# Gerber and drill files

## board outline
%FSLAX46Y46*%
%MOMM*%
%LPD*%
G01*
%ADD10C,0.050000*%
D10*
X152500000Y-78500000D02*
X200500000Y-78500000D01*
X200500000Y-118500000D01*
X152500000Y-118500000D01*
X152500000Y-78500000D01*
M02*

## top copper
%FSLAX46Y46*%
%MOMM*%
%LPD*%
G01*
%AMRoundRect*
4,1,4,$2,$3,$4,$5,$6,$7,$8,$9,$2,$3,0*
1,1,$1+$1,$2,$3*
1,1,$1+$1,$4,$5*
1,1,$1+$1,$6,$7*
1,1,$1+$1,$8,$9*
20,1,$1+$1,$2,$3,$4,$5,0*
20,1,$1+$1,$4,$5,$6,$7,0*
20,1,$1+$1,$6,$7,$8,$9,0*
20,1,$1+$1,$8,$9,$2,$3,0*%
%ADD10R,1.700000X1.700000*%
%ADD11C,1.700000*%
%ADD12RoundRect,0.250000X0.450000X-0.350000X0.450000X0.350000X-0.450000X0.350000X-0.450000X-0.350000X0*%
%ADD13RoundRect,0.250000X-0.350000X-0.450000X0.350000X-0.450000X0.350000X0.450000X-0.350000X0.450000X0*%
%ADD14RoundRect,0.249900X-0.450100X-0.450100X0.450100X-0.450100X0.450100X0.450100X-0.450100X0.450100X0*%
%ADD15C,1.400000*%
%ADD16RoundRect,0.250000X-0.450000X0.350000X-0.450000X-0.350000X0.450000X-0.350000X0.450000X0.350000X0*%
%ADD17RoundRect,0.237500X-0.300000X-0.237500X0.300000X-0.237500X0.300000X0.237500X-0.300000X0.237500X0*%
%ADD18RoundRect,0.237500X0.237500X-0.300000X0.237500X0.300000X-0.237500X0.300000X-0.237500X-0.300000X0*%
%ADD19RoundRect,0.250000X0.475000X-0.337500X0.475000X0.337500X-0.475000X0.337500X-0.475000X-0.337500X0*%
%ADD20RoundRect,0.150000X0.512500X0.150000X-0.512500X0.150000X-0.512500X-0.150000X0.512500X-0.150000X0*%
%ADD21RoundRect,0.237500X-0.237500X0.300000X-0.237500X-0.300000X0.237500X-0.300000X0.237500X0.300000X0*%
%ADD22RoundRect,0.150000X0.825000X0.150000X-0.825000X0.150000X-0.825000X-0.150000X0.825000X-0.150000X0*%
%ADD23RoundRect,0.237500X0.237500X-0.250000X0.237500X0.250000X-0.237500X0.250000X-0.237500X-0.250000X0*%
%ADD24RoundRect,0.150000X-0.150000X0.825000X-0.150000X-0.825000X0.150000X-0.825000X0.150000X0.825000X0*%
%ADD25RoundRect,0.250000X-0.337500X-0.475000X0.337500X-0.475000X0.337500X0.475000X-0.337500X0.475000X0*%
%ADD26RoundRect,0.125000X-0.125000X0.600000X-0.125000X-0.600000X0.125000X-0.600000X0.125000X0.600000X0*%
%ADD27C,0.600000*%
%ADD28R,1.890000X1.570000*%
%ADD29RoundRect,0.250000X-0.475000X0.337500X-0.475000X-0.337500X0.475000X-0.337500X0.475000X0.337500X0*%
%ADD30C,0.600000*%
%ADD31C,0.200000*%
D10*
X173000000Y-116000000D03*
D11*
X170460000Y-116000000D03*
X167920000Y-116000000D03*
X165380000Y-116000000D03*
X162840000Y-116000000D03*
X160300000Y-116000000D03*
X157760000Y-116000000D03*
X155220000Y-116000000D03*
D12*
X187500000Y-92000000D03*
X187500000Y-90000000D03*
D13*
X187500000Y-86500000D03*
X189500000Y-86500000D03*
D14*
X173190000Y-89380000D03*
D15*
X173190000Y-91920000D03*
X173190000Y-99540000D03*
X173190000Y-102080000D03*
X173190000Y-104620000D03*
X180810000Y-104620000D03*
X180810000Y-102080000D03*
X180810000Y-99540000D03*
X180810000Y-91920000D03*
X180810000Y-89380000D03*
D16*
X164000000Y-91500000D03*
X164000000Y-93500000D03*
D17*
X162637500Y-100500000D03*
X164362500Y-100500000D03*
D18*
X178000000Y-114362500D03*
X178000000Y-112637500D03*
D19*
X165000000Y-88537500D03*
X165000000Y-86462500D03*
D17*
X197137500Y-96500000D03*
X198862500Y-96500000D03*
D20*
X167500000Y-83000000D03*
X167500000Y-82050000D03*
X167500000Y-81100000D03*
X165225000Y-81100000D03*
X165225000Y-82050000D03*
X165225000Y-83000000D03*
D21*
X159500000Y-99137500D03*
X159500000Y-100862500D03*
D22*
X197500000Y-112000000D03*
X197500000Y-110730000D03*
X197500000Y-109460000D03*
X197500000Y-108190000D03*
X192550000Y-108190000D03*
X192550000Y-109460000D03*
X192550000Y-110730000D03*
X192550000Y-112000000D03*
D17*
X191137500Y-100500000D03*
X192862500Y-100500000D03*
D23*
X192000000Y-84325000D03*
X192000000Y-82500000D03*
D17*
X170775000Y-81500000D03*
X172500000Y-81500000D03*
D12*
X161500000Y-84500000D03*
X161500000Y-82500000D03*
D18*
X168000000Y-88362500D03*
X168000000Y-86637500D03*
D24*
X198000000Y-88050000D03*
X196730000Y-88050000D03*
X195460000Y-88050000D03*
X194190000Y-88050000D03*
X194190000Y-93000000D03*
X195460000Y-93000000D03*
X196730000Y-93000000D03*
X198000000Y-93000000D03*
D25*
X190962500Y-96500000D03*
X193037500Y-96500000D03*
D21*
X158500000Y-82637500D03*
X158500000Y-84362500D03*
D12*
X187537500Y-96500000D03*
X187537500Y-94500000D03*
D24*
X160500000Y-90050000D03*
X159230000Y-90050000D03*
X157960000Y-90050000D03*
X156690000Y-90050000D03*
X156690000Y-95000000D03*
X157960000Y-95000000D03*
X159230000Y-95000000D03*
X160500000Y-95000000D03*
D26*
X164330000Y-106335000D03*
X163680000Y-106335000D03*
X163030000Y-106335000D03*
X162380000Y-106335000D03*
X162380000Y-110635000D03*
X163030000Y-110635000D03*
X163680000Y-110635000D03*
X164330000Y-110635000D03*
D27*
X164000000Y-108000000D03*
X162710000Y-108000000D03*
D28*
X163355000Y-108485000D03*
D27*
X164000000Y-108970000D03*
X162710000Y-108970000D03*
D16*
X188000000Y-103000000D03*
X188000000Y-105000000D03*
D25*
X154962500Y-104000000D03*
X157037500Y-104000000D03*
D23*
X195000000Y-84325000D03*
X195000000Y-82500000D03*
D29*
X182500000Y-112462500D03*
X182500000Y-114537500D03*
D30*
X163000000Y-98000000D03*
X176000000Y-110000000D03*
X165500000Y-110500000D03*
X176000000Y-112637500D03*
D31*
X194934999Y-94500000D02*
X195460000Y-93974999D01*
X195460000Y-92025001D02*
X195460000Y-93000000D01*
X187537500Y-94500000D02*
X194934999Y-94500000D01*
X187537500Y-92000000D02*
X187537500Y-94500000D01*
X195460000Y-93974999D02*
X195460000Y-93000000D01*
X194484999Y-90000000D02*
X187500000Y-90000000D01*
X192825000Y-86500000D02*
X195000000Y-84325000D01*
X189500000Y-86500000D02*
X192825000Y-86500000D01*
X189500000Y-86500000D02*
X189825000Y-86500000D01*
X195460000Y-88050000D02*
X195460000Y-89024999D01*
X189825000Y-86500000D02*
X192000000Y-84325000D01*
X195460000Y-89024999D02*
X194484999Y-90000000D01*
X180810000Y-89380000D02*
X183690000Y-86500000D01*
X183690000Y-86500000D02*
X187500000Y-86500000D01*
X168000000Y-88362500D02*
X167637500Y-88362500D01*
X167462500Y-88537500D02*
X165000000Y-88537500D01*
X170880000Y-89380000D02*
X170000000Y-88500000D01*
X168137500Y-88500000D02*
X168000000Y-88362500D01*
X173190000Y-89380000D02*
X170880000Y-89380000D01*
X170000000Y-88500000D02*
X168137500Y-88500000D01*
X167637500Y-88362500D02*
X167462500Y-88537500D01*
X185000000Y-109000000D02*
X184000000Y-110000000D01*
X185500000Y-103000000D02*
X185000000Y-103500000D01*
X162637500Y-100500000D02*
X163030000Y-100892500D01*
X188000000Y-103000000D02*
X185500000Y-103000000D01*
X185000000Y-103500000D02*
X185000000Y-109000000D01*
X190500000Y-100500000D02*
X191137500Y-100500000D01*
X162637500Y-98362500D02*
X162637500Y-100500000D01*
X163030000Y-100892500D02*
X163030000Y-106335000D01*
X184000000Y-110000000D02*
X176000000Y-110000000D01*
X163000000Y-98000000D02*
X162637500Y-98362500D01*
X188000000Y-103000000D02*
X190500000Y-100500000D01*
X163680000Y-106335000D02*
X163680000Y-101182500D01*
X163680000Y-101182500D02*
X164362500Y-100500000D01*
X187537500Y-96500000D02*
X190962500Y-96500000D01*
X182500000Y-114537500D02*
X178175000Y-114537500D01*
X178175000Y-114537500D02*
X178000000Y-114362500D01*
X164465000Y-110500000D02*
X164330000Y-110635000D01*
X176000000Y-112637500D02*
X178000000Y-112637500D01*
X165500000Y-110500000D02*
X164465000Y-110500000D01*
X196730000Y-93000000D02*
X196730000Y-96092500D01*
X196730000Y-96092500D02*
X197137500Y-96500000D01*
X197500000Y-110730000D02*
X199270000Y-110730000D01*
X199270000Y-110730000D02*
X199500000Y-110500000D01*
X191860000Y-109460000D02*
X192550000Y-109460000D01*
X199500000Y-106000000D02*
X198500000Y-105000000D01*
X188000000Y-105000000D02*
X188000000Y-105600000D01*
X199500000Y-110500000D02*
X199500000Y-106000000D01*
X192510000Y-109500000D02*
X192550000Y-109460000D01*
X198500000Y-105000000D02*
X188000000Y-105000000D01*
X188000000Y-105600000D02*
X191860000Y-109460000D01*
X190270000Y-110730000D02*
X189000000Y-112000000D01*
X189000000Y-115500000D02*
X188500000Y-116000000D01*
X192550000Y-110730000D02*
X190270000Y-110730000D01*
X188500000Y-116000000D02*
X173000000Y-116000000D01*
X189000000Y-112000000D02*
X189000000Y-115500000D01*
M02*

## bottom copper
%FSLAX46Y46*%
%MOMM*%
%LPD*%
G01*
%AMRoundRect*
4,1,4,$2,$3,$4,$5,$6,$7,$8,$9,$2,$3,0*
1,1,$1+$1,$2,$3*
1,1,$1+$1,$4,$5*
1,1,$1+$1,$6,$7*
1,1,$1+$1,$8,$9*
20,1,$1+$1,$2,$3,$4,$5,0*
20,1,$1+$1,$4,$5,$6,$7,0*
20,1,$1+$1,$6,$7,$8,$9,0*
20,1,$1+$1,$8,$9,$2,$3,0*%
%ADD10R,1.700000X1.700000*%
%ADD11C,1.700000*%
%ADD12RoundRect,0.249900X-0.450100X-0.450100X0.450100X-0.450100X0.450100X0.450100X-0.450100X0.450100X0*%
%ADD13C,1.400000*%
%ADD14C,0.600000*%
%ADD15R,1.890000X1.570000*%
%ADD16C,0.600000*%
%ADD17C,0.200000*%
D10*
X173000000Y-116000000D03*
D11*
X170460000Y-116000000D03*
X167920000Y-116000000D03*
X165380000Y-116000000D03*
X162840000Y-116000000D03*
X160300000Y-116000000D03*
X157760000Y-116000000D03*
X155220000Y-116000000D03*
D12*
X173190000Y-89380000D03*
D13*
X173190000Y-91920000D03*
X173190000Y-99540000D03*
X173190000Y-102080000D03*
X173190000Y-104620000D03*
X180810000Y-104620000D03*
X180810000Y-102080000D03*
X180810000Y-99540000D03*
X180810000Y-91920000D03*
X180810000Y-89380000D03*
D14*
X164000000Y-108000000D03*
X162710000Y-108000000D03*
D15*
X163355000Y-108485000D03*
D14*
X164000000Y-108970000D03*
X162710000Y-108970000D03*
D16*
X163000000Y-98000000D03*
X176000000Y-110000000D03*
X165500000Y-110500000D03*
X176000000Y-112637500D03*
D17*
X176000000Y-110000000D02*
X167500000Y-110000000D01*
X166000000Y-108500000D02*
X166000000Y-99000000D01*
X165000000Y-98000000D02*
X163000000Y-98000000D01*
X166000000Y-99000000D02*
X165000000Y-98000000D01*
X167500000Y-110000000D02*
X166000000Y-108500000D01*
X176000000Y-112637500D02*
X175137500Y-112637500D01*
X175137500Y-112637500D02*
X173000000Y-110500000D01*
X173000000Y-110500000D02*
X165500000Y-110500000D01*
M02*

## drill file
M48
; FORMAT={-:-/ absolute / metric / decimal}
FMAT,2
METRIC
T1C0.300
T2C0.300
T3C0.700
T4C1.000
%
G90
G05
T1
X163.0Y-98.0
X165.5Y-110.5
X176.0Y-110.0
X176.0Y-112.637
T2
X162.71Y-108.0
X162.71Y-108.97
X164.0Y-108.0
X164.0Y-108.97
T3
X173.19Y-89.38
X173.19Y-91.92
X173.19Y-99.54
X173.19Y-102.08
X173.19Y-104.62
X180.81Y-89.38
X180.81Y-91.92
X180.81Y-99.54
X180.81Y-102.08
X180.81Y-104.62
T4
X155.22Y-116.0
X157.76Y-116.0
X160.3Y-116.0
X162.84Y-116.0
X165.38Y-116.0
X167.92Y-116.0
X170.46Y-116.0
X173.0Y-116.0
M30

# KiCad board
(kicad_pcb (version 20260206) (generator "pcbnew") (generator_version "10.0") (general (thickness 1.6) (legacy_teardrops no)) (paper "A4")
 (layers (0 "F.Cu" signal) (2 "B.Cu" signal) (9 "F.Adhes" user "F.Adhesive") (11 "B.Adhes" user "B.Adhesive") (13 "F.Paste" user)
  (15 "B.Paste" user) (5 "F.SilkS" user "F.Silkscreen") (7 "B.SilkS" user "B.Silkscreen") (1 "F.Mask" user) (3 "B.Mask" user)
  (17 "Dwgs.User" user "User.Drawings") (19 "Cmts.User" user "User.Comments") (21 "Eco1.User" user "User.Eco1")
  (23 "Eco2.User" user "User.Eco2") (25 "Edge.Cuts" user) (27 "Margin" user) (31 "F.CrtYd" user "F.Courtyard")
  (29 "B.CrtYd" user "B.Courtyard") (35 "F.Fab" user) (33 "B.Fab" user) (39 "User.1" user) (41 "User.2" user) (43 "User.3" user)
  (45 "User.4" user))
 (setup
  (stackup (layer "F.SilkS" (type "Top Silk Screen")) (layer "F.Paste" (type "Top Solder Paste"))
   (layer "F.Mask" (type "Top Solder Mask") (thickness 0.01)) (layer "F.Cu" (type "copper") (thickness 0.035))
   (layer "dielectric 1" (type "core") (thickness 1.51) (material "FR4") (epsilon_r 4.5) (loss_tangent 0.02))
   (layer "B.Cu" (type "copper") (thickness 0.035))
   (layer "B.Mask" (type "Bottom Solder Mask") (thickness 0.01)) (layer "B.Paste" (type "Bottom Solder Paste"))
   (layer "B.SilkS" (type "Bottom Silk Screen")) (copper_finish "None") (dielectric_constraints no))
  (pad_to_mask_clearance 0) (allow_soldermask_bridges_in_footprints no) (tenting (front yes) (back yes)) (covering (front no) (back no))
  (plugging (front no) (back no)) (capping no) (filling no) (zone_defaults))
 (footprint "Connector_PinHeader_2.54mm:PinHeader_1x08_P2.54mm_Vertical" (layer "F.Cu") (at 173 116 -90)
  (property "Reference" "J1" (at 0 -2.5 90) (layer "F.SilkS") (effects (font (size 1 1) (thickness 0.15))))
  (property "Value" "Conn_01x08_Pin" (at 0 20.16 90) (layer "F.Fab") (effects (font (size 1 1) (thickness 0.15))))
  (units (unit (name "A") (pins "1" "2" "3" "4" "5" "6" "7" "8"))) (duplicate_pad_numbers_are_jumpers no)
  (pad "1" thru_hole rect (at 0 0 270) (size 1.7 1.7) (drill 1) (layers "*.Cu" "*.Mask") (remove_unused_layers no) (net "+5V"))
  (pad "2" thru_hole circle (at 0 2.54 270) (size 1.7 1.7) (drill 1) (layers "*.Cu" "*.Mask") (remove_unused_layers no) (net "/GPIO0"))
  (pad "3" thru_hole circle (at 0 5.08 270) (size 1.7 1.7) (drill 1) (layers "*.Cu" "*.Mask") (remove_unused_layers no) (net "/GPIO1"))
  (pad "4" thru_hole circle (at 0 7.62 270) (size 1.7 1.7) (drill 1) (layers "*.Cu" "*.Mask") (remove_unused_layers no) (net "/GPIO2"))
  (pad "5" thru_hole circle (at 0 10.16 270) (size 1.7 1.7) (drill 1) (layers "*.Cu" "*.Mask") (remove_unused_layers no) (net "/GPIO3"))
  (pad "6" thru_hole circle (at 0 12.7 270) (size 1.7 1.7) (drill 1) (layers "*.Cu" "*.Mask") (remove_unused_layers no) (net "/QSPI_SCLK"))
  (pad "7" thru_hole circle (at 0 15.24 270) (size 1.7 1.7) (drill 1) (layers "*.Cu" "*.Mask") (remove_unused_layers no) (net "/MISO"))
  (pad "8" thru_hole circle (at 0 17.78 270) (size 1.7 1.7) (drill 1) (layers "*.Cu" "*.Mask") (remove_unused_layers no) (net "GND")))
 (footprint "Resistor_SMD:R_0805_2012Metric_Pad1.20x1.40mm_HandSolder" (layer "F.Cu") (at 187.5 91 90)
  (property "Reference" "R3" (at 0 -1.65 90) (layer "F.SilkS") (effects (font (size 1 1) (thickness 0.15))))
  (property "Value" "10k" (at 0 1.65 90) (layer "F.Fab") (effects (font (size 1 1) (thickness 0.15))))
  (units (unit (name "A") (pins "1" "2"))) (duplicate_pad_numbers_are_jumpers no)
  (pad "1" smd roundrect (at -1 0 90) (size 1.2 1.4) (layers "F.Cu" "F.Mask" "F.Paste") (roundrect_rratio 0.208333) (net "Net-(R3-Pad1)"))
  (pad "2" smd roundrect (at 1 0 90) (size 1.2 1.4) (layers "F.Cu" "F.Mask" "F.Paste") (roundrect_rratio 0.208333) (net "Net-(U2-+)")))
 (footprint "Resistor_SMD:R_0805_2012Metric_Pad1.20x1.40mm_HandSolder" (layer "F.Cu") (at 188.5 86.5)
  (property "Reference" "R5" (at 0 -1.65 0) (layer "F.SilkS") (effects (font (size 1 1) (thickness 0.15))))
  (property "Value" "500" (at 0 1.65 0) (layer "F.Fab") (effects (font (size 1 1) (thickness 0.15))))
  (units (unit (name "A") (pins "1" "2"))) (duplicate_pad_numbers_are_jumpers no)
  (pad "1" smd roundrect (at -1 0) (size 1.2 1.4) (layers "F.Cu" "F.Mask" "F.Paste") (roundrect_rratio 0.208333) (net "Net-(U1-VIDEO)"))
  (pad "2" smd roundrect (at 1 0) (size 1.2 1.4) (layers "F.Cu" "F.Mask" "F.Paste") (roundrect_rratio 0.208333) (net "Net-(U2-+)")))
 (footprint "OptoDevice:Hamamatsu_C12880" (layer "F.Cu") (at 173.19 89.38)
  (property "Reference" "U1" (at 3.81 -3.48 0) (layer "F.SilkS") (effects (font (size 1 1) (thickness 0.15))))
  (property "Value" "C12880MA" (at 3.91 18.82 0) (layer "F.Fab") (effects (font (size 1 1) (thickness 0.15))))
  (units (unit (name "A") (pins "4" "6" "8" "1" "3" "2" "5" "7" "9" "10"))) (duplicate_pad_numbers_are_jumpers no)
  (pad "1" thru_hole roundrect (at 0 0) (size 1.4 1.4) (drill 0.7) (layers "*.Cu" "*.Mask") (remove_unused_layers no)
   (roundrect_rratio 0.1785) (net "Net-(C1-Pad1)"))
  (pad "2" thru_hole circle (at 0 2.54) (size 1.4 1.4) (drill 0.7) (layers "*.Cu" "*.Mask") (remove_unused_layers no) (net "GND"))
  (pad "3" thru_hole circle (at 0 10.16) (size 1.4 1.4) (drill 0.7) (layers "*.Cu" "*.Mask") (remove_unused_layers no) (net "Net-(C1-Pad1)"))
  (pad "4" thru_hole circle (at 0 12.7) (size 1.4 1.4) (drill 0.7) (layers "*.Cu" "*.Mask") (remove_unused_layers no) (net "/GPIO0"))
  (pad "5" thru_hole circle (at 0 15.24) (size 1.4 1.4) (drill 0.7) (layers "*.Cu" "*.Mask") (remove_unused_layers no) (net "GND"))
  (pad "6" thru_hole circle (at 7.62 15.24) (size 1.4 1.4) (drill 0.7) (layers "*.Cu" "*.Mask") (remove_unused_layers no) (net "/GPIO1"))
  (pad "7" thru_hole circle (at 7.62 12.7) (size 1.4 1.4) (drill 0.7) (layers "*.Cu" "*.Mask") (remove_unused_layers no) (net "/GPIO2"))
  (pad "8" thru_hole circle (at 7.62 10.16) (size 1.4 1.4) (drill 0.7) (layers "*.Cu" "*.Mask") (remove_unused_layers no)
   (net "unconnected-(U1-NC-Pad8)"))
  (pad "9" thru_hole circle (at 7.62 2.54) (size 1.4 1.4) (drill 0.7) (layers "*.Cu" "*.Mask") (remove_unused_layers no) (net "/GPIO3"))
  (pad "10" thru_hole circle (at 7.62 0) (size 1.4 1.4) (drill 0.7) (layers "*.Cu" "*.Mask") (remove_unused_layers no)
   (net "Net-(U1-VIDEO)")))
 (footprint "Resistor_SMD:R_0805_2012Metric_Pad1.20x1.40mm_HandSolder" (layer "F.Cu") (at 164 92.5 -90)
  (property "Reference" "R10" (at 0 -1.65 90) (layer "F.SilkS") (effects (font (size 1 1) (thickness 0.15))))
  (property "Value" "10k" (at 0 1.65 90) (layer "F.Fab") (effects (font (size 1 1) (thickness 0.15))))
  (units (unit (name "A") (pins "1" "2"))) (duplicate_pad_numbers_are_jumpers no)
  (pad "1" smd roundrect (at -1 0 270) (size 1.2 1.4) (layers "F.Cu" "F.Mask" "F.Paste") (roundrect_rratio 0.208333) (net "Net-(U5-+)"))
  (pad "2" smd roundrect (at 1 0 270) (size 1.2 1.4) (layers "F.Cu" "F.Mask" "F.Paste") (roundrect_rratio 0.208333) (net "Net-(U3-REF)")))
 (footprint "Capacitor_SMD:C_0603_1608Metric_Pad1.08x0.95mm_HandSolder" (layer "F.Cu") (at 163.5 100.5)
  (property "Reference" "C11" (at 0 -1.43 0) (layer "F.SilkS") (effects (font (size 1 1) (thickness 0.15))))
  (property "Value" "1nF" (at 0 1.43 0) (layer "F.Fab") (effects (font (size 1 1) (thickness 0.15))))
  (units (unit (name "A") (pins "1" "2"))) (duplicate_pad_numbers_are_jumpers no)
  (pad "1" smd roundrect (at -0.8625 0) (size 1.075 0.95) (layers "F.Cu" "F.Mask" "F.Paste") (roundrect_rratio 0.25) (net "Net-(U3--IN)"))
  (pad "2" smd roundrect (at 0.8625 0) (size 1.075 0.95) (layers "F.Cu" "F.Mask" "F.Paste") (roundrect_rratio 0.25) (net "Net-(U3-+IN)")))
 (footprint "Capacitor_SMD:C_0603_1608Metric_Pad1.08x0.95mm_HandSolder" (layer "F.Cu") (at 178 113.5 90)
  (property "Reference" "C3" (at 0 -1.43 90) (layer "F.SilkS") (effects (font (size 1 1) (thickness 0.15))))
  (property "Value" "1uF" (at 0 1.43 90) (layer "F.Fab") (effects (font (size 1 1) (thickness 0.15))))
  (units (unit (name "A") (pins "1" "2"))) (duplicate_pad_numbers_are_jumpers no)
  (pad "1" smd roundrect (at -0.8625 0 90) (size 1.075 0.95) (layers "F.Cu" "F.Mask" "F.Paste") (roundrect_rratio 0.25)
   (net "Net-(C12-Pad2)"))
  (pad "2" smd roundrect (at 0.8625 0 90) (size 1.075 0.95) (layers "F.Cu" "F.Mask" "F.Paste") (roundrect_rratio 0.25) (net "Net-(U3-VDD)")))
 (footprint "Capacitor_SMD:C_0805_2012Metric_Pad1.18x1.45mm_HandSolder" (layer "F.Cu") (at 165 87.5 90)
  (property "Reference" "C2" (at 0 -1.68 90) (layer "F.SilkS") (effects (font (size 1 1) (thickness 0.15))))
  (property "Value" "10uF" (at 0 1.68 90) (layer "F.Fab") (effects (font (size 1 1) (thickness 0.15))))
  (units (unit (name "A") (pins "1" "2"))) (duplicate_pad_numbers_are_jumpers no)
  (pad "1" smd roundrect (at -1.0375 0 90) (size 1.175 1.45) (layers "F.Cu" "F.Mask" "F.Paste") (roundrect_rratio 0.212766)
   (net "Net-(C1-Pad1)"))
  (pad "2" smd roundrect (at 1.0375 0 90) (size 1.175 1.45) (layers "F.Cu" "F.Mask" "F.Paste") (roundrect_rratio 0.212766) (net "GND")))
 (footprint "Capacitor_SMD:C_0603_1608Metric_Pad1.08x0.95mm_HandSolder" (layer "F.Cu") (at 198 96.5)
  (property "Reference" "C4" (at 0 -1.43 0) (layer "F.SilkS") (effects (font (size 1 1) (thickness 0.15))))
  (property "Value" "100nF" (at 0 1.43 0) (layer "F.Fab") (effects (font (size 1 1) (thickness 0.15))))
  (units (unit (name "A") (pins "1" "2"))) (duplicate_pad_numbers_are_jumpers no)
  (pad "1" smd roundrect (at -0.8625 0) (size 1.075 0.95) (layers "F.Cu" "F.Mask" "F.Paste") (roundrect_rratio 0.25) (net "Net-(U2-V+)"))
  (pad "2" smd roundrect (at 0.8625 0) (size 1.075 0.95) (layers "F.Cu" "F.Mask" "F.Paste") (roundrect_rratio 0.25) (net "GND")))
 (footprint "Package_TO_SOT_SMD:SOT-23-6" (layer "F.Cu") (at 166.3625 82.05 180)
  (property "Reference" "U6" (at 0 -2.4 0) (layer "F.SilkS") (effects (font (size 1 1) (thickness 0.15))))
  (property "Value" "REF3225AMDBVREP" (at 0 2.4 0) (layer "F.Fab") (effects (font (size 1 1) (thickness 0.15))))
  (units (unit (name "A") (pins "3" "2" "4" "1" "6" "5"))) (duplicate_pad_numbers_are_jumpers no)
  (pad "1" smd roundrect (at -1.1375 -0.95 180) (size 1.325 0.6) (layers "F.Cu" "F.Mask" "F.Paste") (roundrect_rratio 0.25) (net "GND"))
  (pad "2" smd roundrect (at -1.1375 0 180) (size 1.325 0.6) (layers "F.Cu" "F.Mask" "F.Paste") (roundrect_rratio 0.25) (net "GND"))
  (pad "3" smd roundrect (at -1.1375 0.95 180) (size 1.325 0.6) (layers "F.Cu" "F.Mask" "F.Paste") (roundrect_rratio 0.25)
   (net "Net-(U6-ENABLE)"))
  (pad "4" smd roundrect (at 1.1375 0.95 180) (size 1.325 0.6) (layers "F.Cu" "F.Mask" "F.Paste") (roundrect_rratio 0.25) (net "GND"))
  (pad "5" smd roundrect (at 1.1375 0 180) (size 1.325 0.6) (layers "F.Cu" "F.Mask" "F.Paste") (roundrect_rratio 0.25)
   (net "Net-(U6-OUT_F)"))
  (pad "6" smd roundrect (at 1.1375 -0.95 180) (size 1.325 0.6) (layers "F.Cu" "F.Mask" "F.Paste") (roundrect_rratio 0.25)
   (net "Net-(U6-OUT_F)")))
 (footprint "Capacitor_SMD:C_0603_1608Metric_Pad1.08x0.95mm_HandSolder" (layer "F.Cu") (at 159.5 100 -90)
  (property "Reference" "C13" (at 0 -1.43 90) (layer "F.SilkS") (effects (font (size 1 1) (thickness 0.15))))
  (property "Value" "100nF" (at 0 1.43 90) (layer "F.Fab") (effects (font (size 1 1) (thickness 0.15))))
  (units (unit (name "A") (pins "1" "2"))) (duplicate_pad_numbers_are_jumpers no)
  (pad "1" smd roundrect (at -0.8625 0 270) (size 1.075 0.95) (layers "F.Cu" "F.Mask" "F.Paste") (roundrect_rratio 0.25) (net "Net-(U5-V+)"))
  (pad "2" smd roundrect (at 0.8625 0 270) (size 1.075 0.95) (layers "F.Cu" "F.Mask" "F.Paste") (roundrect_rratio 0.25) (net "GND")))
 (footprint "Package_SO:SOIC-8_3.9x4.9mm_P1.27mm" (layer "F.Cu") (at 195.025 110.095 180)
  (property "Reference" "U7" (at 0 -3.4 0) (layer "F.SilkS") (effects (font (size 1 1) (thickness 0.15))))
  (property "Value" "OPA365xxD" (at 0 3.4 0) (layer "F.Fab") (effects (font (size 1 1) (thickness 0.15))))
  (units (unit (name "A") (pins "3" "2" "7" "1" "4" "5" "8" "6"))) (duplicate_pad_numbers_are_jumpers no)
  (pad "1" smd roundrect (at -2.475 -1.905 180) (size 1.95 0.6) (layers "F.Cu" "F.Mask" "F.Paste") (roundrect_rratio 0.25)
   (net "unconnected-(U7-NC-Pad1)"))
  (pad "2" smd roundrect (at -2.475 -0.635 180) (size 1.95 0.6) (layers "F.Cu" "F.Mask" "F.Paste") (roundrect_rratio 0.25)
   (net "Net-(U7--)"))
  (pad "3" smd roundrect (at -2.475 0.635 180) (size 1.95 0.6) (layers "F.Cu" "F.Mask" "F.Paste") (roundrect_rratio 0.25) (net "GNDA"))
  (pad "4" smd roundrect (at -2.475 1.905 180) (size 1.95 0.6) (layers "F.Cu" "F.Mask" "F.Paste") (roundrect_rratio 0.25) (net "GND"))
  (pad "5" smd roundrect (at 2.475 1.905 180) (size 1.95 0.6) (layers "F.Cu" "F.Mask" "F.Paste") (roundrect_rratio 0.25)
   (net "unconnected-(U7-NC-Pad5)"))
  (pad "6" smd roundrect (at 2.475 0.635 180) (size 1.95 0.6) (layers "F.Cu" "F.Mask" "F.Paste") (roundrect_rratio 0.25) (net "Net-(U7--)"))
  (pad "7" smd roundrect (at 2.475 -0.635 180) (size 1.95 0.6) (layers "F.Cu" "F.Mask" "F.Paste") (roundrect_rratio 0.25) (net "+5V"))
  (pad "8" smd roundrect (at 2.475 -1.905 180) (size 1.95 0.6) (layers "F.Cu" "F.Mask" "F.Paste") (roundrect_rratio 0.25)
   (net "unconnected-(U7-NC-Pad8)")))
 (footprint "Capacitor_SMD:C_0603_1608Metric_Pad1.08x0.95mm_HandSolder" (layer "F.Cu") (at 192 100.5)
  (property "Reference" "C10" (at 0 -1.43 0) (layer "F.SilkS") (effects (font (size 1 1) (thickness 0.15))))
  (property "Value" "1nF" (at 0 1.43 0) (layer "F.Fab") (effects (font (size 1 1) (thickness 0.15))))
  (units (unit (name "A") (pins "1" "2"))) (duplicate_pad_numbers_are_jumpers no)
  (pad "1" smd roundrect (at -0.8625 0) (size 1.075 0.95) (layers "F.Cu" "F.Mask" "F.Paste") (roundrect_rratio 0.25) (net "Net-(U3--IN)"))
  (pad "2" smd roundrect (at 0.8625 0) (size 1.075 0.95) (layers "F.Cu" "F.Mask" "F.Paste") (roundrect_rratio 0.25) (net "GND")))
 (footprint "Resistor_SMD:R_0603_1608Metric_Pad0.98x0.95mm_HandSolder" (layer "F.Cu") (at 192 83.4125 90)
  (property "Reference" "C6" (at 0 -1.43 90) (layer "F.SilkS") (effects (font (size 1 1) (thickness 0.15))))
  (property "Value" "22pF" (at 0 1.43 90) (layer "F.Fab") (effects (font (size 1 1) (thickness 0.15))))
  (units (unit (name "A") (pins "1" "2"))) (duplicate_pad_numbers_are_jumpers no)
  (pad "1" smd roundrect (at -0.9125 0 90) (size 0.975 0.95) (layers "F.Cu" "F.Mask" "F.Paste") (roundrect_rratio 0.25) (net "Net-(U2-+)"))
  (pad "2" smd roundrect (at 0.9125 0 90) (size 0.975 0.95) (layers "F.Cu" "F.Mask" "F.Paste") (roundrect_rratio 0.25) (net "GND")))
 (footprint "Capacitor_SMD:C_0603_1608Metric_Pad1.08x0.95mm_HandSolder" (layer "F.Cu") (at 171.6375 81.5)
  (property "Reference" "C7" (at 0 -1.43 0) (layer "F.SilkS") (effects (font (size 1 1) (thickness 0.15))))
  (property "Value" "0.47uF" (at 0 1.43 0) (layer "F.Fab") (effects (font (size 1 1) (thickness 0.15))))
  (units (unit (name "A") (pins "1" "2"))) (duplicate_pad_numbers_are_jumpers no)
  (pad "1" smd roundrect (at -0.8625 0) (size 1.075 0.95) (layers "F.Cu" "F.Mask" "F.Paste") (roundrect_rratio 0.25) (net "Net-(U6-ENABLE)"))
  (pad "2" smd roundrect (at 0.8625 0) (size 1.075 0.95) (layers "F.Cu" "F.Mask" "F.Paste") (roundrect_rratio 0.25) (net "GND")))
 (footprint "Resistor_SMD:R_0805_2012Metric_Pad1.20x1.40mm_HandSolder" (layer "F.Cu") (at 161.5 83.5 90)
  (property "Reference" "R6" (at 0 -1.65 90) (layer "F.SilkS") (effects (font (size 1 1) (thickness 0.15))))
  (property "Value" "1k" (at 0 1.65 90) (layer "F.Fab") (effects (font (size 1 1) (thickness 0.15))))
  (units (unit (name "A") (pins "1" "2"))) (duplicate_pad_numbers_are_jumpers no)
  (pad "1" smd roundrect (at -1 0 90) (size 1.2 1.4) (layers "F.Cu" "F.Mask" "F.Paste") (roundrect_rratio 0.208333) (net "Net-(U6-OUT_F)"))
  (pad "2" smd roundrect (at 1 0 90) (size 1.2 1.4) (layers "F.Cu" "F.Mask" "F.Paste") (roundrect_rratio 0.208333) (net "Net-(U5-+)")))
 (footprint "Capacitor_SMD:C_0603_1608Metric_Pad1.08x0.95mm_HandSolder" (layer "F.Cu") (at 168 87.5 90)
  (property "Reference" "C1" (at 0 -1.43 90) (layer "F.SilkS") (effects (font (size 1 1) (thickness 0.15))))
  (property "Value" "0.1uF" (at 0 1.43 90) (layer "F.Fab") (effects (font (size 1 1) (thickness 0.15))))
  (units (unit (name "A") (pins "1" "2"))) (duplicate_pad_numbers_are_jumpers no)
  (pad "1" smd roundrect (at -0.8625 0 90) (size 1.075 0.95) (layers "F.Cu" "F.Mask" "F.Paste") (roundrect_rratio 0.25)
   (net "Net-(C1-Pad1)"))
  (pad "2" smd roundrect (at 0.8625 0 90) (size 1.075 0.95) (layers "F.Cu" "F.Mask" "F.Paste") (roundrect_rratio 0.25) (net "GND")))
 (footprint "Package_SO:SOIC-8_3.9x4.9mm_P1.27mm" (layer "F.Cu") (at 196.095 90.525 -90)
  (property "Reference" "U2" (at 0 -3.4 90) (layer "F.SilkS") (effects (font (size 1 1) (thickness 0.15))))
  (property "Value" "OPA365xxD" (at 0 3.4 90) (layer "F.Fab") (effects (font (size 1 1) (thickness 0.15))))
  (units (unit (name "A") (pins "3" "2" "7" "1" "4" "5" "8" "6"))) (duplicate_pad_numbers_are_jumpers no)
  (pad "1" smd roundrect (at -2.475 -1.905 270) (size 1.95 0.6) (layers "F.Cu" "F.Mask" "F.Paste") (roundrect_rratio 0.25)
   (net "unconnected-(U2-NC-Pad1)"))
  (pad "2" smd roundrect (at -2.475 -0.635 270) (size 1.95 0.6) (layers "F.Cu" "F.Mask" "F.Paste") (roundrect_rratio 0.25) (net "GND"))
  (pad "3" smd roundrect (at -2.475 0.635 270) (size 1.95 0.6) (layers "F.Cu" "F.Mask" "F.Paste") (roundrect_rratio 0.25) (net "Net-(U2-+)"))
  (pad "4" smd roundrect (at -2.475 1.905 270) (size 1.95 0.6) (layers "F.Cu" "F.Mask" "F.Paste") (roundrect_rratio 0.25) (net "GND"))
  (pad "5" smd roundrect (at 2.475 1.905 270) (size 1.95 0.6) (layers "F.Cu" "F.Mask" "F.Paste") (roundrect_rratio 0.25)
   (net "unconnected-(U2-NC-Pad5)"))
  (pad "6" smd roundrect (at 2.475 0.635 270) (size 1.95 0.6) (layers "F.Cu" "F.Mask" "F.Paste") (roundrect_rratio 0.25)
   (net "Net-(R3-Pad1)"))
  (pad "7" smd roundrect (at 2.475 -0.635 270) (size 1.95 0.6) (layers "F.Cu" "F.Mask" "F.Paste") (roundrect_rratio 0.25)
   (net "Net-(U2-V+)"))
  (pad "8" smd roundrect (at 2.475 -1.905 270) (size 1.95 0.6) (layers "F.Cu" "F.Mask" "F.Paste") (roundrect_rratio 0.25)
   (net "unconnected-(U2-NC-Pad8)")))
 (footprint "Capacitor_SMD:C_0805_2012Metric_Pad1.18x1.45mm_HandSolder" (layer "F.Cu") (at 192 96.5)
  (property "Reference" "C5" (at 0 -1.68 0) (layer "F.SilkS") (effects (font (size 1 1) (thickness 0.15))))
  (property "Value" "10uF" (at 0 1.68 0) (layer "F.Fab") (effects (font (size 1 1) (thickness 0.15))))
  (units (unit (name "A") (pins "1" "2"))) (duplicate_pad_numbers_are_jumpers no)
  (pad "1" smd roundrect (at -1.0375 0) (size 1.175 1.45) (layers "F.Cu" "F.Mask" "F.Paste") (roundrect_rratio 0.212766)
   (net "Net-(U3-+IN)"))
  (pad "2" smd roundrect (at 1.0375 0) (size 1.175 1.45) (layers "F.Cu" "F.Mask" "F.Paste") (roundrect_rratio 0.212766) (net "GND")))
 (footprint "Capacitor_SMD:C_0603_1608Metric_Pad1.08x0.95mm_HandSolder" (layer "F.Cu") (at 158.5 83.5 -90)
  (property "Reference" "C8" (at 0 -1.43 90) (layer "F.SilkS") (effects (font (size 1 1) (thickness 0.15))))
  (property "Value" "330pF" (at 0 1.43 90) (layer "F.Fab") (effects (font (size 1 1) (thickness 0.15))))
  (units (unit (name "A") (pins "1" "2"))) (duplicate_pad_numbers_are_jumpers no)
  (pad "1" smd roundrect (at -0.8625 0 270) (size 1.075 0.95) (layers "F.Cu" "F.Mask" "F.Paste") (roundrect_rratio 0.25) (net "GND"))
  (pad "2" smd roundrect (at 0.8625 0 270) (size 1.075 0.95) (layers "F.Cu" "F.Mask" "F.Paste") (roundrect_rratio 0.25) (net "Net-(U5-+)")))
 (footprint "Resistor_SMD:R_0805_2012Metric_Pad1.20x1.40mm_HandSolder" (layer "F.Cu") (at 187.5375 95.5 90)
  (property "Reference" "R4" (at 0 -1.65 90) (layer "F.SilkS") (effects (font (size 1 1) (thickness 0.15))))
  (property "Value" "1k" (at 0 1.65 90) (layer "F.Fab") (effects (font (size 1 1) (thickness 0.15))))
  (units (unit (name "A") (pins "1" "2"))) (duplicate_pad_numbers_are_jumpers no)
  (pad "1" smd roundrect (at -1 0 90) (size 1.2 1.4) (layers "F.Cu" "F.Mask" "F.Paste") (roundrect_rratio 0.208333) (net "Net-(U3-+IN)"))
  (pad "2" smd roundrect (at 1 0 90) (size 1.2 1.4) (layers "F.Cu" "F.Mask" "F.Paste") (roundrect_rratio 0.208333) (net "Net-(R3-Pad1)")))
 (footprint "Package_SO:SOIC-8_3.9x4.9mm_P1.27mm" (layer "F.Cu") (at 158.595 92.525 -90)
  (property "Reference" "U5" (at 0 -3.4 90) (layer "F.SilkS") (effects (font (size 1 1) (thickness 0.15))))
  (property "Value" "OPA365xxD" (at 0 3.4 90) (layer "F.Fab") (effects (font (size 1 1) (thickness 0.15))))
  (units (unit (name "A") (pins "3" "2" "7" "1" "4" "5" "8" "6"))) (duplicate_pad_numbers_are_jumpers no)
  (pad "1" smd roundrect (at -2.475 -1.905 270) (size 1.95 0.6) (layers "F.Cu" "F.Mask" "F.Paste") (roundrect_rratio 0.25)
   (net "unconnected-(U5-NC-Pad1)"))
  (pad "2" smd roundrect (at -2.475 -0.635 270) (size 1.95 0.6) (layers "F.Cu" "F.Mask" "F.Paste") (roundrect_rratio 0.25) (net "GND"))
  (pad "3" smd roundrect (at -2.475 0.635 270) (size 1.95 0.6) (layers "F.Cu" "F.Mask" "F.Paste") (roundrect_rratio 0.25) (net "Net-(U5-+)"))
  (pad "4" smd roundrect (at -2.475 1.905 270) (size 1.95 0.6) (layers "F.Cu" "F.Mask" "F.Paste") (roundrect_rratio 0.25) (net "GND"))
  (pad "5" smd roundrect (at 2.475 1.905 270) (size 1.95 0.6) (layers "F.Cu" "F.Mask" "F.Paste") (roundrect_rratio 0.25)
   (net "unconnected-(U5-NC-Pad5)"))
  (pad "6" smd roundrect (at 2.475 0.635 270) (size 1.95 0.6) (layers "F.Cu" "F.Mask" "F.Paste") (roundrect_rratio 0.25)
   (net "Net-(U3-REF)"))
  (pad "7" smd roundrect (at 2.475 -0.635 270) (size 1.95 0.6) (layers "F.Cu" "F.Mask" "F.Paste") (roundrect_rratio 0.25)
   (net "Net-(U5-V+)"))
  (pad "8" smd roundrect (at 2.475 -1.905 270) (size 1.95 0.6) (layers "F.Cu" "F.Mask" "F.Paste") (roundrect_rratio 0.25)
   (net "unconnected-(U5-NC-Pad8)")))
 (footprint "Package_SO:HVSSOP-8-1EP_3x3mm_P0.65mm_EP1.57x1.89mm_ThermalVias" (layer "F.Cu") (at 163.355 108.485 -90)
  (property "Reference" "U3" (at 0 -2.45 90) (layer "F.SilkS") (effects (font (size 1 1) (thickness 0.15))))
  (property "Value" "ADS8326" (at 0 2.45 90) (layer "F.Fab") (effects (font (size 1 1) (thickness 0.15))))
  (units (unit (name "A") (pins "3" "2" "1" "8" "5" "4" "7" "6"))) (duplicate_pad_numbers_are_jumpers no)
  (pad "" smd roundrect (at -0.39 -0.47 270) (size 0.63 0.76) (layers "F.Paste") (roundrect_rratio 0.25))
  (pad "" smd roundrect (at -0.39 0.47 270) (size 0.63 0.76) (layers "F.Paste") (roundrect_rratio 0.25))
  (pad "" smd roundrect (at 0.39 -0.47 270) (size 0.63 0.76) (layers "F.Paste") (roundrect_rratio 0.25))
  (pad "" smd roundrect (at 0.39 0.47 270) (size 0.63 0.76) (layers "F.Paste") (roundrect_rratio 0.25))
  (pad "1" smd roundrect (at -2.15 -0.975 270) (size 1.45 0.5) (layers "F.Cu" "F.Mask" "F.Paste") (roundrect_rratio 0.25)
   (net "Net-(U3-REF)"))
  (pad "2" smd roundrect (at -2.15 -0.325 270) (size 1.45 0.5) (layers "F.Cu" "F.Mask" "F.Paste") (roundrect_rratio 0.25)
   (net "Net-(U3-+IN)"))
  (pad "3" smd roundrect (at -2.15 0.325 270) (size 1.45 0.5) (layers "F.Cu" "F.Mask" "F.Paste") (roundrect_rratio 0.25)
   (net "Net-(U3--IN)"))
  (pad "4" smd roundrect (at -2.15 0.975 270) (size 1.45 0.5) (layers "F.Cu" "F.Mask" "F.Paste") (roundrect_rratio 0.25) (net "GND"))
  (pad "5" smd roundrect (at 2.15 0.975 270) (size 1.45 0.5) (layers "F.Cu" "F.Mask" "F.Paste") (roundrect_rratio 0.25) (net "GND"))
  (pad "6" smd roundrect (at 2.15 0.325 270) (size 1.45 0.5) (layers "F.Cu" "F.Mask" "F.Paste") (roundrect_rratio 0.25) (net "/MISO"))
  (pad "7" smd roundrect (at 2.15 -0.325 270) (size 1.45 0.5) (layers "F.Cu" "F.Mask" "F.Paste") (roundrect_rratio 0.25) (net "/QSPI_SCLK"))
  (pad "8" smd roundrect (at 2.15 -0.975 270) (size 1.45 0.5) (layers "F.Cu" "F.Mask" "F.Paste") (roundrect_rratio 0.25)
   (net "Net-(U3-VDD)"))
  (pad "9" thru_hole circle (at -0.485 -0.645 270) (size 0.6 0.6) (drill 0.3) (layers "*.Cu") (remove_unused_layers no))
  (pad "9" thru_hole circle (at -0.485 0.645 270) (size 0.6 0.6) (drill 0.3) (layers "*.Cu") (remove_unused_layers no))
  (pad "9" smd rect (at 0 0 270) (size 1.57 1.89) (layers "F.Cu" "F.Mask") (zone_connect 2))
  (pad "9" smd rect (at 0 0 270) (size 1.57 1.89) (layers "B.Cu") (zone_connect 2))
  (pad "9" thru_hole circle (at 0.485 -0.645 270) (size 0.6 0.6) (drill 0.3) (layers "*.Cu") (remove_unused_layers no))
  (pad "9" thru_hole circle (at 0.485 0.645 270) (size 0.6 0.6) (drill 0.3) (layers "*.Cu") (remove_unused_layers no)))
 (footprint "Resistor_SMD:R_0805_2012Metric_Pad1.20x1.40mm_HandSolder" (layer "F.Cu") (at 188 104 -90)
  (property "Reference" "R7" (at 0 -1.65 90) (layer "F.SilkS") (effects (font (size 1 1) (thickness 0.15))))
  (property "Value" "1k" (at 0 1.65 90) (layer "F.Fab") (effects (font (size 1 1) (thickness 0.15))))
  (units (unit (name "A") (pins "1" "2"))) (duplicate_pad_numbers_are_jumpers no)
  (pad "1" smd roundrect (at -1 0 270) (size 1.2 1.4) (layers "F.Cu" "F.Mask" "F.Paste") (roundrect_rratio 0.208333) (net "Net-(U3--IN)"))
  (pad "2" smd roundrect (at 1 0 270) (size 1.2 1.4) (layers "F.Cu" "F.Mask" "F.Paste") (roundrect_rratio 0.208333) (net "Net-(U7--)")))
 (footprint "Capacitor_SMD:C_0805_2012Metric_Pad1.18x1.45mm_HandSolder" (layer "F.Cu") (at 156 104)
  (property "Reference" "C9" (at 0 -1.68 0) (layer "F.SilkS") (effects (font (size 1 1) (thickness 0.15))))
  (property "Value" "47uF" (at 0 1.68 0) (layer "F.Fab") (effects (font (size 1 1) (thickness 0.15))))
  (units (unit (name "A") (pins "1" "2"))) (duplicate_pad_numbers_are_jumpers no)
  (pad "1" smd roundrect (at -1.0375 0) (size 1.175 1.45) (layers "F.Cu" "F.Mask" "F.Paste") (roundrect_rratio 0.212766) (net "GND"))
  (pad "2" smd roundrect (at 1.0375 0) (size 1.175 1.45) (layers "F.Cu" "F.Mask" "F.Paste") (roundrect_rratio 0.212766) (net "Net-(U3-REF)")))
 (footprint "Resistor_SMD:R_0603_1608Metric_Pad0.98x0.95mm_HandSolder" (layer "F.Cu") (at 195 83.4125 90)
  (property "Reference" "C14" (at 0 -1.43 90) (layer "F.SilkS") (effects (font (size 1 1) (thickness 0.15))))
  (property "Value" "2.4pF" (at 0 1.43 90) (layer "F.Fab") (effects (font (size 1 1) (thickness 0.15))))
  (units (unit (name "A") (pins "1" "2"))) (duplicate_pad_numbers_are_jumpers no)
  (pad "1" smd roundrect (at -0.9125 0 90) (size 0.975 0.95) (layers "F.Cu" "F.Mask" "F.Paste") (roundrect_rratio 0.25) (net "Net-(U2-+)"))
  (pad "2" smd roundrect (at 0.9125 0 90) (size 0.975 0.95) (layers "F.Cu" "F.Mask" "F.Paste") (roundrect_rratio 0.25) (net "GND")))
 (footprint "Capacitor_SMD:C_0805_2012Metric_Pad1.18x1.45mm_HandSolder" (layer "F.Cu") (at 182.5 113.5 -90)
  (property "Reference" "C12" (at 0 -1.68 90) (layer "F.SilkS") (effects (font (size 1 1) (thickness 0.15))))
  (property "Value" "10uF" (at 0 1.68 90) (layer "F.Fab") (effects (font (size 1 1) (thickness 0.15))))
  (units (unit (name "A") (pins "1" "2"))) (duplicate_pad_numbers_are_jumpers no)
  (pad "1" smd roundrect (at -1.0375 0 270) (size 1.175 1.45) (layers "F.Cu" "F.Mask" "F.Paste") (roundrect_rratio 0.212766) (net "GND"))
  (pad "2" smd roundrect (at 1.0375 0 270) (size 1.175 1.45) (layers "F.Cu" "F.Mask" "F.Paste") (roundrect_rratio 0.212766)
   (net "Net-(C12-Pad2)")))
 (gr_rect (start 152.5 78.5) (end 200.5 118.5) (stroke (width 0.05) (type default)) (fill no) (layer "Edge.Cuts"))
 (segment (start 194.934999 94.5) (end 195.46 93.974999) (width 0.2) (layer "F.Cu") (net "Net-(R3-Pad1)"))
 (segment (start 195.46 92.025001) (end 195.46 93) (width 0.2) (layer "F.Cu") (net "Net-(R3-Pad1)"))
 (segment (start 187.5375 94.5) (end 194.934999 94.5) (width 0.2) (layer "F.Cu") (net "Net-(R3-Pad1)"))
 (segment (start 187.5375 92) (end 187.5375 94.5) (width 0.2) (layer "F.Cu") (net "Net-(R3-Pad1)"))
 (segment (start 195.46 93.974999) (end 195.46 93) (width 0.2) (layer "F.Cu") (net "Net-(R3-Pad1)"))
 (segment (start 194.484999 90) (end 187.5 90) (width 0.2) (layer "F.Cu") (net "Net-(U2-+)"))
 (segment (start 192.825 86.5) (end 195 84.325) (width 0.2) (layer "F.Cu") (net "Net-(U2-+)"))
 (segment (start 189.5 86.5) (end 192.825 86.5) (width 0.2) (layer "F.Cu") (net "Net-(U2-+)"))
 (segment (start 189.5 86.5) (end 189.825 86.5) (width 0.2) (layer "F.Cu") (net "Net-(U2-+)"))
 (segment (start 195.46 88.05) (end 195.46 89.024999) (width 0.2) (layer "F.Cu") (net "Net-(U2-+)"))
 (segment (start 189.825 86.5) (end 192 84.325) (width 0.2) (layer "F.Cu") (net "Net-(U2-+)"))
 (segment (start 195.46 89.024999) (end 194.484999 90) (width 0.2) (layer "F.Cu") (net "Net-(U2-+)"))
 (segment (start 180.81 89.38) (end 183.69 86.5) (width 0.2) (layer "F.Cu") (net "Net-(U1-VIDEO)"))
 (segment (start 183.69 86.5) (end 187.5 86.5) (width 0.2) (layer "F.Cu") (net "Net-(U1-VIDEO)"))
 (segment (start 168 88.3625) (end 167.6375 88.3625) (width 0.2) (layer "F.Cu") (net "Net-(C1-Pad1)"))
 (segment (start 167.4625 88.5375) (end 165 88.5375) (width 0.2) (layer "F.Cu") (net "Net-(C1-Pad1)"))
 (segment (start 170.88 89.38) (end 170 88.5) (width 0.2) (layer "F.Cu") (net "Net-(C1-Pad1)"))
 (segment (start 168.1375 88.5) (end 168 88.3625) (width 0.2) (layer "F.Cu") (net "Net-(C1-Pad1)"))
 (segment (start 173.19 89.38) (end 170.88 89.38) (width 0.2) (layer "F.Cu") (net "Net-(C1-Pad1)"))
 (segment (start 170 88.5) (end 168.1375 88.5) (width 0.2) (layer "F.Cu") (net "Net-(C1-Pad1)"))
 (segment (start 167.6375 88.3625) (end 167.4625 88.5375) (width 0.2) (layer "F.Cu") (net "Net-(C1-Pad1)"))
 (segment (start 185 109) (end 184 110) (width 0.2) (layer "F.Cu") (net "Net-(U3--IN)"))
 (segment (start 185.5 103) (end 185 103.5) (width 0.2) (layer "F.Cu") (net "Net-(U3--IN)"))
 (segment (start 162.6375 100.5) (end 163.03 100.8925) (width 0.2) (layer "F.Cu") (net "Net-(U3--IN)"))
 (segment (start 188 103) (end 185.5 103) (width 0.2) (layer "F.Cu") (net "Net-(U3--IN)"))
 (segment (start 185 103.5) (end 185 109) (width 0.2) (layer "F.Cu") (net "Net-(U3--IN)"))
 (segment (start 190.5 100.5) (end 191.1375 100.5) (width 0.2) (layer "F.Cu") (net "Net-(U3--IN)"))
 (segment (start 162.6375 98.3625) (end 162.6375 100.5) (width 0.2) (layer "F.Cu") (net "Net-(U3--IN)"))
 (segment (start 163.03 100.8925) (end 163.03 106.335) (width 0.2) (layer "F.Cu") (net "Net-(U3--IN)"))
 (segment (start 184 110) (end 176 110) (width 0.2) (layer "F.Cu") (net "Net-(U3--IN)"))
 (segment (start 163 98) (end 162.6375 98.3625) (width 0.2) (layer "F.Cu") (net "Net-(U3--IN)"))
 (segment (start 188 103) (end 190.5 100.5) (width 0.2) (layer "F.Cu") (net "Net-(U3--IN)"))
 (via (at 163 98) (size 0.6) (drill 0.3) (layers "F.Cu" "B.Cu") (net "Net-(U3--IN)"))
 (via (at 176 110) (size 0.6) (drill 0.3) (layers "F.Cu" "B.Cu") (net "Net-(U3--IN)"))
 (segment (start 176 110) (end 167.5 110) (width 0.2) (layer "B.Cu") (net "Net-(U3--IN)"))
 (segment (start 166 108.5) (end 166 99) (width 0.2) (layer "B.Cu") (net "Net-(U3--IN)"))
 (segment (start 165 98) (end 163 98) (width 0.2) (layer "B.Cu") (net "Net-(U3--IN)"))
 (segment (start 166 99) (end 165 98) (width 0.2) (layer "B.Cu") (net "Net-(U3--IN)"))
 (segment (start 167.5 110) (end 166 108.5) (width 0.2) (layer "B.Cu") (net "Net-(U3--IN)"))
 (segment (start 163.68 106.335) (end 163.68 101.1825) (width 0.2) (layer "F.Cu") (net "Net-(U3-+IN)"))
 (segment (start 163.68 101.1825) (end 164.3625 100.5) (width 0.2) (layer "F.Cu") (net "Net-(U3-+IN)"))
 (segment (start 187.5375 96.5) (end 190.9625 96.5) (width 0.2) (layer "F.Cu") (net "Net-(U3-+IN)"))
 (segment (start 182.5 114.5375) (end 178.175 114.5375) (width 0.2) (layer "F.Cu") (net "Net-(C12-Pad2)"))
 (segment (start 178.175 114.5375) (end 178 114.3625) (width 0.2) (layer "F.Cu") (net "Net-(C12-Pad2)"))
 (segment (start 164.465 110.5) (end 164.33 110.635) (width 0.2) (layer "F.Cu") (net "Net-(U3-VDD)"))
 (segment (start 176 112.6375) (end 178 112.6375) (width 0.2) (layer "F.Cu") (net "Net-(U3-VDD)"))
 (segment (start 165.5 110.5) (end 164.465 110.5) (width 0.2) (layer "F.Cu") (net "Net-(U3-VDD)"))
 (via (at 165.5 110.5) (size 0.6) (drill 0.3) (layers "F.Cu" "B.Cu") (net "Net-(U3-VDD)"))
 (via (at 176 112.6375) (size 0.6) (drill 0.3) (layers "F.Cu" "B.Cu") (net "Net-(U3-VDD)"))
 (segment (start 176 112.6375) (end 175.1375 112.6375) (width 0.2) (layer "B.Cu") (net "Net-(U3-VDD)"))
 (segment (start 175.1375 112.6375) (end 173 110.5) (width 0.2) (layer "B.Cu") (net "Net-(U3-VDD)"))
 (segment (start 173 110.5) (end 165.5 110.5) (width 0.2) (layer "B.Cu") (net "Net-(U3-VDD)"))
 (segment (start 196.73 93) (end 196.73 96.0925) (width 0.2) (layer "F.Cu") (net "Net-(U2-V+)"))
 (segment (start 196.73 96.0925) (end 197.1375 96.5) (width 0.2) (layer "F.Cu") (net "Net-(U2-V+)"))
 (segment (start 197.5 110.73) (end 199.27 110.73) (width 0.2) (layer "F.Cu") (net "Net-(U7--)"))
 (segment (start 199.27 110.73) (end 199.5 110.5) (width 0.2) (layer "F.Cu") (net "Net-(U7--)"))
 (segment (start 191.86 109.46) (end 192.55 109.46) (width 0.2) (layer "F.Cu") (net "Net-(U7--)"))
 (segment (start 199.5 106) (end 198.5 105) (width 0.2) (layer "F.Cu") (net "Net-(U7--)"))
 (segment (start 188 105) (end 188 105.6) (width 0.2) (layer "F.Cu") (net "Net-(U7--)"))
 (segment (start 199.5 110.5) (end 199.5 106) (width 0.2) (layer "F.Cu") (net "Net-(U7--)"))
 (segment (start 192.51 109.5) (end 192.55 109.46) (width 0.2) (layer "F.Cu") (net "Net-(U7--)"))
 (segment (start 198.5 105) (end 188 105) (width 0.2) (layer "F.Cu") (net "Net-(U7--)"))
 (segment (start 188 105.6) (end 191.86 109.46) (width 0.2) (layer "F.Cu") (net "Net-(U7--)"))
 (segment (start 190.27 110.73) (end 189 112) (width 0.2) (layer "F.Cu") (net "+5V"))
 (segment (start 189 115.5) (end 188.5 116) (width 0.2) (layer "F.Cu") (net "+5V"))
 (segment (start 192.55 110.73) (end 190.27 110.73) (width 0.2) (layer "F.Cu") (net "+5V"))
 (segment (start 188.5 116) (end 173 116) (width 0.2) (layer "F.Cu") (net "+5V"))
 (segment (start 189 112) (end 189 115.5) (width 0.2) (layer "F.Cu") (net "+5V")))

